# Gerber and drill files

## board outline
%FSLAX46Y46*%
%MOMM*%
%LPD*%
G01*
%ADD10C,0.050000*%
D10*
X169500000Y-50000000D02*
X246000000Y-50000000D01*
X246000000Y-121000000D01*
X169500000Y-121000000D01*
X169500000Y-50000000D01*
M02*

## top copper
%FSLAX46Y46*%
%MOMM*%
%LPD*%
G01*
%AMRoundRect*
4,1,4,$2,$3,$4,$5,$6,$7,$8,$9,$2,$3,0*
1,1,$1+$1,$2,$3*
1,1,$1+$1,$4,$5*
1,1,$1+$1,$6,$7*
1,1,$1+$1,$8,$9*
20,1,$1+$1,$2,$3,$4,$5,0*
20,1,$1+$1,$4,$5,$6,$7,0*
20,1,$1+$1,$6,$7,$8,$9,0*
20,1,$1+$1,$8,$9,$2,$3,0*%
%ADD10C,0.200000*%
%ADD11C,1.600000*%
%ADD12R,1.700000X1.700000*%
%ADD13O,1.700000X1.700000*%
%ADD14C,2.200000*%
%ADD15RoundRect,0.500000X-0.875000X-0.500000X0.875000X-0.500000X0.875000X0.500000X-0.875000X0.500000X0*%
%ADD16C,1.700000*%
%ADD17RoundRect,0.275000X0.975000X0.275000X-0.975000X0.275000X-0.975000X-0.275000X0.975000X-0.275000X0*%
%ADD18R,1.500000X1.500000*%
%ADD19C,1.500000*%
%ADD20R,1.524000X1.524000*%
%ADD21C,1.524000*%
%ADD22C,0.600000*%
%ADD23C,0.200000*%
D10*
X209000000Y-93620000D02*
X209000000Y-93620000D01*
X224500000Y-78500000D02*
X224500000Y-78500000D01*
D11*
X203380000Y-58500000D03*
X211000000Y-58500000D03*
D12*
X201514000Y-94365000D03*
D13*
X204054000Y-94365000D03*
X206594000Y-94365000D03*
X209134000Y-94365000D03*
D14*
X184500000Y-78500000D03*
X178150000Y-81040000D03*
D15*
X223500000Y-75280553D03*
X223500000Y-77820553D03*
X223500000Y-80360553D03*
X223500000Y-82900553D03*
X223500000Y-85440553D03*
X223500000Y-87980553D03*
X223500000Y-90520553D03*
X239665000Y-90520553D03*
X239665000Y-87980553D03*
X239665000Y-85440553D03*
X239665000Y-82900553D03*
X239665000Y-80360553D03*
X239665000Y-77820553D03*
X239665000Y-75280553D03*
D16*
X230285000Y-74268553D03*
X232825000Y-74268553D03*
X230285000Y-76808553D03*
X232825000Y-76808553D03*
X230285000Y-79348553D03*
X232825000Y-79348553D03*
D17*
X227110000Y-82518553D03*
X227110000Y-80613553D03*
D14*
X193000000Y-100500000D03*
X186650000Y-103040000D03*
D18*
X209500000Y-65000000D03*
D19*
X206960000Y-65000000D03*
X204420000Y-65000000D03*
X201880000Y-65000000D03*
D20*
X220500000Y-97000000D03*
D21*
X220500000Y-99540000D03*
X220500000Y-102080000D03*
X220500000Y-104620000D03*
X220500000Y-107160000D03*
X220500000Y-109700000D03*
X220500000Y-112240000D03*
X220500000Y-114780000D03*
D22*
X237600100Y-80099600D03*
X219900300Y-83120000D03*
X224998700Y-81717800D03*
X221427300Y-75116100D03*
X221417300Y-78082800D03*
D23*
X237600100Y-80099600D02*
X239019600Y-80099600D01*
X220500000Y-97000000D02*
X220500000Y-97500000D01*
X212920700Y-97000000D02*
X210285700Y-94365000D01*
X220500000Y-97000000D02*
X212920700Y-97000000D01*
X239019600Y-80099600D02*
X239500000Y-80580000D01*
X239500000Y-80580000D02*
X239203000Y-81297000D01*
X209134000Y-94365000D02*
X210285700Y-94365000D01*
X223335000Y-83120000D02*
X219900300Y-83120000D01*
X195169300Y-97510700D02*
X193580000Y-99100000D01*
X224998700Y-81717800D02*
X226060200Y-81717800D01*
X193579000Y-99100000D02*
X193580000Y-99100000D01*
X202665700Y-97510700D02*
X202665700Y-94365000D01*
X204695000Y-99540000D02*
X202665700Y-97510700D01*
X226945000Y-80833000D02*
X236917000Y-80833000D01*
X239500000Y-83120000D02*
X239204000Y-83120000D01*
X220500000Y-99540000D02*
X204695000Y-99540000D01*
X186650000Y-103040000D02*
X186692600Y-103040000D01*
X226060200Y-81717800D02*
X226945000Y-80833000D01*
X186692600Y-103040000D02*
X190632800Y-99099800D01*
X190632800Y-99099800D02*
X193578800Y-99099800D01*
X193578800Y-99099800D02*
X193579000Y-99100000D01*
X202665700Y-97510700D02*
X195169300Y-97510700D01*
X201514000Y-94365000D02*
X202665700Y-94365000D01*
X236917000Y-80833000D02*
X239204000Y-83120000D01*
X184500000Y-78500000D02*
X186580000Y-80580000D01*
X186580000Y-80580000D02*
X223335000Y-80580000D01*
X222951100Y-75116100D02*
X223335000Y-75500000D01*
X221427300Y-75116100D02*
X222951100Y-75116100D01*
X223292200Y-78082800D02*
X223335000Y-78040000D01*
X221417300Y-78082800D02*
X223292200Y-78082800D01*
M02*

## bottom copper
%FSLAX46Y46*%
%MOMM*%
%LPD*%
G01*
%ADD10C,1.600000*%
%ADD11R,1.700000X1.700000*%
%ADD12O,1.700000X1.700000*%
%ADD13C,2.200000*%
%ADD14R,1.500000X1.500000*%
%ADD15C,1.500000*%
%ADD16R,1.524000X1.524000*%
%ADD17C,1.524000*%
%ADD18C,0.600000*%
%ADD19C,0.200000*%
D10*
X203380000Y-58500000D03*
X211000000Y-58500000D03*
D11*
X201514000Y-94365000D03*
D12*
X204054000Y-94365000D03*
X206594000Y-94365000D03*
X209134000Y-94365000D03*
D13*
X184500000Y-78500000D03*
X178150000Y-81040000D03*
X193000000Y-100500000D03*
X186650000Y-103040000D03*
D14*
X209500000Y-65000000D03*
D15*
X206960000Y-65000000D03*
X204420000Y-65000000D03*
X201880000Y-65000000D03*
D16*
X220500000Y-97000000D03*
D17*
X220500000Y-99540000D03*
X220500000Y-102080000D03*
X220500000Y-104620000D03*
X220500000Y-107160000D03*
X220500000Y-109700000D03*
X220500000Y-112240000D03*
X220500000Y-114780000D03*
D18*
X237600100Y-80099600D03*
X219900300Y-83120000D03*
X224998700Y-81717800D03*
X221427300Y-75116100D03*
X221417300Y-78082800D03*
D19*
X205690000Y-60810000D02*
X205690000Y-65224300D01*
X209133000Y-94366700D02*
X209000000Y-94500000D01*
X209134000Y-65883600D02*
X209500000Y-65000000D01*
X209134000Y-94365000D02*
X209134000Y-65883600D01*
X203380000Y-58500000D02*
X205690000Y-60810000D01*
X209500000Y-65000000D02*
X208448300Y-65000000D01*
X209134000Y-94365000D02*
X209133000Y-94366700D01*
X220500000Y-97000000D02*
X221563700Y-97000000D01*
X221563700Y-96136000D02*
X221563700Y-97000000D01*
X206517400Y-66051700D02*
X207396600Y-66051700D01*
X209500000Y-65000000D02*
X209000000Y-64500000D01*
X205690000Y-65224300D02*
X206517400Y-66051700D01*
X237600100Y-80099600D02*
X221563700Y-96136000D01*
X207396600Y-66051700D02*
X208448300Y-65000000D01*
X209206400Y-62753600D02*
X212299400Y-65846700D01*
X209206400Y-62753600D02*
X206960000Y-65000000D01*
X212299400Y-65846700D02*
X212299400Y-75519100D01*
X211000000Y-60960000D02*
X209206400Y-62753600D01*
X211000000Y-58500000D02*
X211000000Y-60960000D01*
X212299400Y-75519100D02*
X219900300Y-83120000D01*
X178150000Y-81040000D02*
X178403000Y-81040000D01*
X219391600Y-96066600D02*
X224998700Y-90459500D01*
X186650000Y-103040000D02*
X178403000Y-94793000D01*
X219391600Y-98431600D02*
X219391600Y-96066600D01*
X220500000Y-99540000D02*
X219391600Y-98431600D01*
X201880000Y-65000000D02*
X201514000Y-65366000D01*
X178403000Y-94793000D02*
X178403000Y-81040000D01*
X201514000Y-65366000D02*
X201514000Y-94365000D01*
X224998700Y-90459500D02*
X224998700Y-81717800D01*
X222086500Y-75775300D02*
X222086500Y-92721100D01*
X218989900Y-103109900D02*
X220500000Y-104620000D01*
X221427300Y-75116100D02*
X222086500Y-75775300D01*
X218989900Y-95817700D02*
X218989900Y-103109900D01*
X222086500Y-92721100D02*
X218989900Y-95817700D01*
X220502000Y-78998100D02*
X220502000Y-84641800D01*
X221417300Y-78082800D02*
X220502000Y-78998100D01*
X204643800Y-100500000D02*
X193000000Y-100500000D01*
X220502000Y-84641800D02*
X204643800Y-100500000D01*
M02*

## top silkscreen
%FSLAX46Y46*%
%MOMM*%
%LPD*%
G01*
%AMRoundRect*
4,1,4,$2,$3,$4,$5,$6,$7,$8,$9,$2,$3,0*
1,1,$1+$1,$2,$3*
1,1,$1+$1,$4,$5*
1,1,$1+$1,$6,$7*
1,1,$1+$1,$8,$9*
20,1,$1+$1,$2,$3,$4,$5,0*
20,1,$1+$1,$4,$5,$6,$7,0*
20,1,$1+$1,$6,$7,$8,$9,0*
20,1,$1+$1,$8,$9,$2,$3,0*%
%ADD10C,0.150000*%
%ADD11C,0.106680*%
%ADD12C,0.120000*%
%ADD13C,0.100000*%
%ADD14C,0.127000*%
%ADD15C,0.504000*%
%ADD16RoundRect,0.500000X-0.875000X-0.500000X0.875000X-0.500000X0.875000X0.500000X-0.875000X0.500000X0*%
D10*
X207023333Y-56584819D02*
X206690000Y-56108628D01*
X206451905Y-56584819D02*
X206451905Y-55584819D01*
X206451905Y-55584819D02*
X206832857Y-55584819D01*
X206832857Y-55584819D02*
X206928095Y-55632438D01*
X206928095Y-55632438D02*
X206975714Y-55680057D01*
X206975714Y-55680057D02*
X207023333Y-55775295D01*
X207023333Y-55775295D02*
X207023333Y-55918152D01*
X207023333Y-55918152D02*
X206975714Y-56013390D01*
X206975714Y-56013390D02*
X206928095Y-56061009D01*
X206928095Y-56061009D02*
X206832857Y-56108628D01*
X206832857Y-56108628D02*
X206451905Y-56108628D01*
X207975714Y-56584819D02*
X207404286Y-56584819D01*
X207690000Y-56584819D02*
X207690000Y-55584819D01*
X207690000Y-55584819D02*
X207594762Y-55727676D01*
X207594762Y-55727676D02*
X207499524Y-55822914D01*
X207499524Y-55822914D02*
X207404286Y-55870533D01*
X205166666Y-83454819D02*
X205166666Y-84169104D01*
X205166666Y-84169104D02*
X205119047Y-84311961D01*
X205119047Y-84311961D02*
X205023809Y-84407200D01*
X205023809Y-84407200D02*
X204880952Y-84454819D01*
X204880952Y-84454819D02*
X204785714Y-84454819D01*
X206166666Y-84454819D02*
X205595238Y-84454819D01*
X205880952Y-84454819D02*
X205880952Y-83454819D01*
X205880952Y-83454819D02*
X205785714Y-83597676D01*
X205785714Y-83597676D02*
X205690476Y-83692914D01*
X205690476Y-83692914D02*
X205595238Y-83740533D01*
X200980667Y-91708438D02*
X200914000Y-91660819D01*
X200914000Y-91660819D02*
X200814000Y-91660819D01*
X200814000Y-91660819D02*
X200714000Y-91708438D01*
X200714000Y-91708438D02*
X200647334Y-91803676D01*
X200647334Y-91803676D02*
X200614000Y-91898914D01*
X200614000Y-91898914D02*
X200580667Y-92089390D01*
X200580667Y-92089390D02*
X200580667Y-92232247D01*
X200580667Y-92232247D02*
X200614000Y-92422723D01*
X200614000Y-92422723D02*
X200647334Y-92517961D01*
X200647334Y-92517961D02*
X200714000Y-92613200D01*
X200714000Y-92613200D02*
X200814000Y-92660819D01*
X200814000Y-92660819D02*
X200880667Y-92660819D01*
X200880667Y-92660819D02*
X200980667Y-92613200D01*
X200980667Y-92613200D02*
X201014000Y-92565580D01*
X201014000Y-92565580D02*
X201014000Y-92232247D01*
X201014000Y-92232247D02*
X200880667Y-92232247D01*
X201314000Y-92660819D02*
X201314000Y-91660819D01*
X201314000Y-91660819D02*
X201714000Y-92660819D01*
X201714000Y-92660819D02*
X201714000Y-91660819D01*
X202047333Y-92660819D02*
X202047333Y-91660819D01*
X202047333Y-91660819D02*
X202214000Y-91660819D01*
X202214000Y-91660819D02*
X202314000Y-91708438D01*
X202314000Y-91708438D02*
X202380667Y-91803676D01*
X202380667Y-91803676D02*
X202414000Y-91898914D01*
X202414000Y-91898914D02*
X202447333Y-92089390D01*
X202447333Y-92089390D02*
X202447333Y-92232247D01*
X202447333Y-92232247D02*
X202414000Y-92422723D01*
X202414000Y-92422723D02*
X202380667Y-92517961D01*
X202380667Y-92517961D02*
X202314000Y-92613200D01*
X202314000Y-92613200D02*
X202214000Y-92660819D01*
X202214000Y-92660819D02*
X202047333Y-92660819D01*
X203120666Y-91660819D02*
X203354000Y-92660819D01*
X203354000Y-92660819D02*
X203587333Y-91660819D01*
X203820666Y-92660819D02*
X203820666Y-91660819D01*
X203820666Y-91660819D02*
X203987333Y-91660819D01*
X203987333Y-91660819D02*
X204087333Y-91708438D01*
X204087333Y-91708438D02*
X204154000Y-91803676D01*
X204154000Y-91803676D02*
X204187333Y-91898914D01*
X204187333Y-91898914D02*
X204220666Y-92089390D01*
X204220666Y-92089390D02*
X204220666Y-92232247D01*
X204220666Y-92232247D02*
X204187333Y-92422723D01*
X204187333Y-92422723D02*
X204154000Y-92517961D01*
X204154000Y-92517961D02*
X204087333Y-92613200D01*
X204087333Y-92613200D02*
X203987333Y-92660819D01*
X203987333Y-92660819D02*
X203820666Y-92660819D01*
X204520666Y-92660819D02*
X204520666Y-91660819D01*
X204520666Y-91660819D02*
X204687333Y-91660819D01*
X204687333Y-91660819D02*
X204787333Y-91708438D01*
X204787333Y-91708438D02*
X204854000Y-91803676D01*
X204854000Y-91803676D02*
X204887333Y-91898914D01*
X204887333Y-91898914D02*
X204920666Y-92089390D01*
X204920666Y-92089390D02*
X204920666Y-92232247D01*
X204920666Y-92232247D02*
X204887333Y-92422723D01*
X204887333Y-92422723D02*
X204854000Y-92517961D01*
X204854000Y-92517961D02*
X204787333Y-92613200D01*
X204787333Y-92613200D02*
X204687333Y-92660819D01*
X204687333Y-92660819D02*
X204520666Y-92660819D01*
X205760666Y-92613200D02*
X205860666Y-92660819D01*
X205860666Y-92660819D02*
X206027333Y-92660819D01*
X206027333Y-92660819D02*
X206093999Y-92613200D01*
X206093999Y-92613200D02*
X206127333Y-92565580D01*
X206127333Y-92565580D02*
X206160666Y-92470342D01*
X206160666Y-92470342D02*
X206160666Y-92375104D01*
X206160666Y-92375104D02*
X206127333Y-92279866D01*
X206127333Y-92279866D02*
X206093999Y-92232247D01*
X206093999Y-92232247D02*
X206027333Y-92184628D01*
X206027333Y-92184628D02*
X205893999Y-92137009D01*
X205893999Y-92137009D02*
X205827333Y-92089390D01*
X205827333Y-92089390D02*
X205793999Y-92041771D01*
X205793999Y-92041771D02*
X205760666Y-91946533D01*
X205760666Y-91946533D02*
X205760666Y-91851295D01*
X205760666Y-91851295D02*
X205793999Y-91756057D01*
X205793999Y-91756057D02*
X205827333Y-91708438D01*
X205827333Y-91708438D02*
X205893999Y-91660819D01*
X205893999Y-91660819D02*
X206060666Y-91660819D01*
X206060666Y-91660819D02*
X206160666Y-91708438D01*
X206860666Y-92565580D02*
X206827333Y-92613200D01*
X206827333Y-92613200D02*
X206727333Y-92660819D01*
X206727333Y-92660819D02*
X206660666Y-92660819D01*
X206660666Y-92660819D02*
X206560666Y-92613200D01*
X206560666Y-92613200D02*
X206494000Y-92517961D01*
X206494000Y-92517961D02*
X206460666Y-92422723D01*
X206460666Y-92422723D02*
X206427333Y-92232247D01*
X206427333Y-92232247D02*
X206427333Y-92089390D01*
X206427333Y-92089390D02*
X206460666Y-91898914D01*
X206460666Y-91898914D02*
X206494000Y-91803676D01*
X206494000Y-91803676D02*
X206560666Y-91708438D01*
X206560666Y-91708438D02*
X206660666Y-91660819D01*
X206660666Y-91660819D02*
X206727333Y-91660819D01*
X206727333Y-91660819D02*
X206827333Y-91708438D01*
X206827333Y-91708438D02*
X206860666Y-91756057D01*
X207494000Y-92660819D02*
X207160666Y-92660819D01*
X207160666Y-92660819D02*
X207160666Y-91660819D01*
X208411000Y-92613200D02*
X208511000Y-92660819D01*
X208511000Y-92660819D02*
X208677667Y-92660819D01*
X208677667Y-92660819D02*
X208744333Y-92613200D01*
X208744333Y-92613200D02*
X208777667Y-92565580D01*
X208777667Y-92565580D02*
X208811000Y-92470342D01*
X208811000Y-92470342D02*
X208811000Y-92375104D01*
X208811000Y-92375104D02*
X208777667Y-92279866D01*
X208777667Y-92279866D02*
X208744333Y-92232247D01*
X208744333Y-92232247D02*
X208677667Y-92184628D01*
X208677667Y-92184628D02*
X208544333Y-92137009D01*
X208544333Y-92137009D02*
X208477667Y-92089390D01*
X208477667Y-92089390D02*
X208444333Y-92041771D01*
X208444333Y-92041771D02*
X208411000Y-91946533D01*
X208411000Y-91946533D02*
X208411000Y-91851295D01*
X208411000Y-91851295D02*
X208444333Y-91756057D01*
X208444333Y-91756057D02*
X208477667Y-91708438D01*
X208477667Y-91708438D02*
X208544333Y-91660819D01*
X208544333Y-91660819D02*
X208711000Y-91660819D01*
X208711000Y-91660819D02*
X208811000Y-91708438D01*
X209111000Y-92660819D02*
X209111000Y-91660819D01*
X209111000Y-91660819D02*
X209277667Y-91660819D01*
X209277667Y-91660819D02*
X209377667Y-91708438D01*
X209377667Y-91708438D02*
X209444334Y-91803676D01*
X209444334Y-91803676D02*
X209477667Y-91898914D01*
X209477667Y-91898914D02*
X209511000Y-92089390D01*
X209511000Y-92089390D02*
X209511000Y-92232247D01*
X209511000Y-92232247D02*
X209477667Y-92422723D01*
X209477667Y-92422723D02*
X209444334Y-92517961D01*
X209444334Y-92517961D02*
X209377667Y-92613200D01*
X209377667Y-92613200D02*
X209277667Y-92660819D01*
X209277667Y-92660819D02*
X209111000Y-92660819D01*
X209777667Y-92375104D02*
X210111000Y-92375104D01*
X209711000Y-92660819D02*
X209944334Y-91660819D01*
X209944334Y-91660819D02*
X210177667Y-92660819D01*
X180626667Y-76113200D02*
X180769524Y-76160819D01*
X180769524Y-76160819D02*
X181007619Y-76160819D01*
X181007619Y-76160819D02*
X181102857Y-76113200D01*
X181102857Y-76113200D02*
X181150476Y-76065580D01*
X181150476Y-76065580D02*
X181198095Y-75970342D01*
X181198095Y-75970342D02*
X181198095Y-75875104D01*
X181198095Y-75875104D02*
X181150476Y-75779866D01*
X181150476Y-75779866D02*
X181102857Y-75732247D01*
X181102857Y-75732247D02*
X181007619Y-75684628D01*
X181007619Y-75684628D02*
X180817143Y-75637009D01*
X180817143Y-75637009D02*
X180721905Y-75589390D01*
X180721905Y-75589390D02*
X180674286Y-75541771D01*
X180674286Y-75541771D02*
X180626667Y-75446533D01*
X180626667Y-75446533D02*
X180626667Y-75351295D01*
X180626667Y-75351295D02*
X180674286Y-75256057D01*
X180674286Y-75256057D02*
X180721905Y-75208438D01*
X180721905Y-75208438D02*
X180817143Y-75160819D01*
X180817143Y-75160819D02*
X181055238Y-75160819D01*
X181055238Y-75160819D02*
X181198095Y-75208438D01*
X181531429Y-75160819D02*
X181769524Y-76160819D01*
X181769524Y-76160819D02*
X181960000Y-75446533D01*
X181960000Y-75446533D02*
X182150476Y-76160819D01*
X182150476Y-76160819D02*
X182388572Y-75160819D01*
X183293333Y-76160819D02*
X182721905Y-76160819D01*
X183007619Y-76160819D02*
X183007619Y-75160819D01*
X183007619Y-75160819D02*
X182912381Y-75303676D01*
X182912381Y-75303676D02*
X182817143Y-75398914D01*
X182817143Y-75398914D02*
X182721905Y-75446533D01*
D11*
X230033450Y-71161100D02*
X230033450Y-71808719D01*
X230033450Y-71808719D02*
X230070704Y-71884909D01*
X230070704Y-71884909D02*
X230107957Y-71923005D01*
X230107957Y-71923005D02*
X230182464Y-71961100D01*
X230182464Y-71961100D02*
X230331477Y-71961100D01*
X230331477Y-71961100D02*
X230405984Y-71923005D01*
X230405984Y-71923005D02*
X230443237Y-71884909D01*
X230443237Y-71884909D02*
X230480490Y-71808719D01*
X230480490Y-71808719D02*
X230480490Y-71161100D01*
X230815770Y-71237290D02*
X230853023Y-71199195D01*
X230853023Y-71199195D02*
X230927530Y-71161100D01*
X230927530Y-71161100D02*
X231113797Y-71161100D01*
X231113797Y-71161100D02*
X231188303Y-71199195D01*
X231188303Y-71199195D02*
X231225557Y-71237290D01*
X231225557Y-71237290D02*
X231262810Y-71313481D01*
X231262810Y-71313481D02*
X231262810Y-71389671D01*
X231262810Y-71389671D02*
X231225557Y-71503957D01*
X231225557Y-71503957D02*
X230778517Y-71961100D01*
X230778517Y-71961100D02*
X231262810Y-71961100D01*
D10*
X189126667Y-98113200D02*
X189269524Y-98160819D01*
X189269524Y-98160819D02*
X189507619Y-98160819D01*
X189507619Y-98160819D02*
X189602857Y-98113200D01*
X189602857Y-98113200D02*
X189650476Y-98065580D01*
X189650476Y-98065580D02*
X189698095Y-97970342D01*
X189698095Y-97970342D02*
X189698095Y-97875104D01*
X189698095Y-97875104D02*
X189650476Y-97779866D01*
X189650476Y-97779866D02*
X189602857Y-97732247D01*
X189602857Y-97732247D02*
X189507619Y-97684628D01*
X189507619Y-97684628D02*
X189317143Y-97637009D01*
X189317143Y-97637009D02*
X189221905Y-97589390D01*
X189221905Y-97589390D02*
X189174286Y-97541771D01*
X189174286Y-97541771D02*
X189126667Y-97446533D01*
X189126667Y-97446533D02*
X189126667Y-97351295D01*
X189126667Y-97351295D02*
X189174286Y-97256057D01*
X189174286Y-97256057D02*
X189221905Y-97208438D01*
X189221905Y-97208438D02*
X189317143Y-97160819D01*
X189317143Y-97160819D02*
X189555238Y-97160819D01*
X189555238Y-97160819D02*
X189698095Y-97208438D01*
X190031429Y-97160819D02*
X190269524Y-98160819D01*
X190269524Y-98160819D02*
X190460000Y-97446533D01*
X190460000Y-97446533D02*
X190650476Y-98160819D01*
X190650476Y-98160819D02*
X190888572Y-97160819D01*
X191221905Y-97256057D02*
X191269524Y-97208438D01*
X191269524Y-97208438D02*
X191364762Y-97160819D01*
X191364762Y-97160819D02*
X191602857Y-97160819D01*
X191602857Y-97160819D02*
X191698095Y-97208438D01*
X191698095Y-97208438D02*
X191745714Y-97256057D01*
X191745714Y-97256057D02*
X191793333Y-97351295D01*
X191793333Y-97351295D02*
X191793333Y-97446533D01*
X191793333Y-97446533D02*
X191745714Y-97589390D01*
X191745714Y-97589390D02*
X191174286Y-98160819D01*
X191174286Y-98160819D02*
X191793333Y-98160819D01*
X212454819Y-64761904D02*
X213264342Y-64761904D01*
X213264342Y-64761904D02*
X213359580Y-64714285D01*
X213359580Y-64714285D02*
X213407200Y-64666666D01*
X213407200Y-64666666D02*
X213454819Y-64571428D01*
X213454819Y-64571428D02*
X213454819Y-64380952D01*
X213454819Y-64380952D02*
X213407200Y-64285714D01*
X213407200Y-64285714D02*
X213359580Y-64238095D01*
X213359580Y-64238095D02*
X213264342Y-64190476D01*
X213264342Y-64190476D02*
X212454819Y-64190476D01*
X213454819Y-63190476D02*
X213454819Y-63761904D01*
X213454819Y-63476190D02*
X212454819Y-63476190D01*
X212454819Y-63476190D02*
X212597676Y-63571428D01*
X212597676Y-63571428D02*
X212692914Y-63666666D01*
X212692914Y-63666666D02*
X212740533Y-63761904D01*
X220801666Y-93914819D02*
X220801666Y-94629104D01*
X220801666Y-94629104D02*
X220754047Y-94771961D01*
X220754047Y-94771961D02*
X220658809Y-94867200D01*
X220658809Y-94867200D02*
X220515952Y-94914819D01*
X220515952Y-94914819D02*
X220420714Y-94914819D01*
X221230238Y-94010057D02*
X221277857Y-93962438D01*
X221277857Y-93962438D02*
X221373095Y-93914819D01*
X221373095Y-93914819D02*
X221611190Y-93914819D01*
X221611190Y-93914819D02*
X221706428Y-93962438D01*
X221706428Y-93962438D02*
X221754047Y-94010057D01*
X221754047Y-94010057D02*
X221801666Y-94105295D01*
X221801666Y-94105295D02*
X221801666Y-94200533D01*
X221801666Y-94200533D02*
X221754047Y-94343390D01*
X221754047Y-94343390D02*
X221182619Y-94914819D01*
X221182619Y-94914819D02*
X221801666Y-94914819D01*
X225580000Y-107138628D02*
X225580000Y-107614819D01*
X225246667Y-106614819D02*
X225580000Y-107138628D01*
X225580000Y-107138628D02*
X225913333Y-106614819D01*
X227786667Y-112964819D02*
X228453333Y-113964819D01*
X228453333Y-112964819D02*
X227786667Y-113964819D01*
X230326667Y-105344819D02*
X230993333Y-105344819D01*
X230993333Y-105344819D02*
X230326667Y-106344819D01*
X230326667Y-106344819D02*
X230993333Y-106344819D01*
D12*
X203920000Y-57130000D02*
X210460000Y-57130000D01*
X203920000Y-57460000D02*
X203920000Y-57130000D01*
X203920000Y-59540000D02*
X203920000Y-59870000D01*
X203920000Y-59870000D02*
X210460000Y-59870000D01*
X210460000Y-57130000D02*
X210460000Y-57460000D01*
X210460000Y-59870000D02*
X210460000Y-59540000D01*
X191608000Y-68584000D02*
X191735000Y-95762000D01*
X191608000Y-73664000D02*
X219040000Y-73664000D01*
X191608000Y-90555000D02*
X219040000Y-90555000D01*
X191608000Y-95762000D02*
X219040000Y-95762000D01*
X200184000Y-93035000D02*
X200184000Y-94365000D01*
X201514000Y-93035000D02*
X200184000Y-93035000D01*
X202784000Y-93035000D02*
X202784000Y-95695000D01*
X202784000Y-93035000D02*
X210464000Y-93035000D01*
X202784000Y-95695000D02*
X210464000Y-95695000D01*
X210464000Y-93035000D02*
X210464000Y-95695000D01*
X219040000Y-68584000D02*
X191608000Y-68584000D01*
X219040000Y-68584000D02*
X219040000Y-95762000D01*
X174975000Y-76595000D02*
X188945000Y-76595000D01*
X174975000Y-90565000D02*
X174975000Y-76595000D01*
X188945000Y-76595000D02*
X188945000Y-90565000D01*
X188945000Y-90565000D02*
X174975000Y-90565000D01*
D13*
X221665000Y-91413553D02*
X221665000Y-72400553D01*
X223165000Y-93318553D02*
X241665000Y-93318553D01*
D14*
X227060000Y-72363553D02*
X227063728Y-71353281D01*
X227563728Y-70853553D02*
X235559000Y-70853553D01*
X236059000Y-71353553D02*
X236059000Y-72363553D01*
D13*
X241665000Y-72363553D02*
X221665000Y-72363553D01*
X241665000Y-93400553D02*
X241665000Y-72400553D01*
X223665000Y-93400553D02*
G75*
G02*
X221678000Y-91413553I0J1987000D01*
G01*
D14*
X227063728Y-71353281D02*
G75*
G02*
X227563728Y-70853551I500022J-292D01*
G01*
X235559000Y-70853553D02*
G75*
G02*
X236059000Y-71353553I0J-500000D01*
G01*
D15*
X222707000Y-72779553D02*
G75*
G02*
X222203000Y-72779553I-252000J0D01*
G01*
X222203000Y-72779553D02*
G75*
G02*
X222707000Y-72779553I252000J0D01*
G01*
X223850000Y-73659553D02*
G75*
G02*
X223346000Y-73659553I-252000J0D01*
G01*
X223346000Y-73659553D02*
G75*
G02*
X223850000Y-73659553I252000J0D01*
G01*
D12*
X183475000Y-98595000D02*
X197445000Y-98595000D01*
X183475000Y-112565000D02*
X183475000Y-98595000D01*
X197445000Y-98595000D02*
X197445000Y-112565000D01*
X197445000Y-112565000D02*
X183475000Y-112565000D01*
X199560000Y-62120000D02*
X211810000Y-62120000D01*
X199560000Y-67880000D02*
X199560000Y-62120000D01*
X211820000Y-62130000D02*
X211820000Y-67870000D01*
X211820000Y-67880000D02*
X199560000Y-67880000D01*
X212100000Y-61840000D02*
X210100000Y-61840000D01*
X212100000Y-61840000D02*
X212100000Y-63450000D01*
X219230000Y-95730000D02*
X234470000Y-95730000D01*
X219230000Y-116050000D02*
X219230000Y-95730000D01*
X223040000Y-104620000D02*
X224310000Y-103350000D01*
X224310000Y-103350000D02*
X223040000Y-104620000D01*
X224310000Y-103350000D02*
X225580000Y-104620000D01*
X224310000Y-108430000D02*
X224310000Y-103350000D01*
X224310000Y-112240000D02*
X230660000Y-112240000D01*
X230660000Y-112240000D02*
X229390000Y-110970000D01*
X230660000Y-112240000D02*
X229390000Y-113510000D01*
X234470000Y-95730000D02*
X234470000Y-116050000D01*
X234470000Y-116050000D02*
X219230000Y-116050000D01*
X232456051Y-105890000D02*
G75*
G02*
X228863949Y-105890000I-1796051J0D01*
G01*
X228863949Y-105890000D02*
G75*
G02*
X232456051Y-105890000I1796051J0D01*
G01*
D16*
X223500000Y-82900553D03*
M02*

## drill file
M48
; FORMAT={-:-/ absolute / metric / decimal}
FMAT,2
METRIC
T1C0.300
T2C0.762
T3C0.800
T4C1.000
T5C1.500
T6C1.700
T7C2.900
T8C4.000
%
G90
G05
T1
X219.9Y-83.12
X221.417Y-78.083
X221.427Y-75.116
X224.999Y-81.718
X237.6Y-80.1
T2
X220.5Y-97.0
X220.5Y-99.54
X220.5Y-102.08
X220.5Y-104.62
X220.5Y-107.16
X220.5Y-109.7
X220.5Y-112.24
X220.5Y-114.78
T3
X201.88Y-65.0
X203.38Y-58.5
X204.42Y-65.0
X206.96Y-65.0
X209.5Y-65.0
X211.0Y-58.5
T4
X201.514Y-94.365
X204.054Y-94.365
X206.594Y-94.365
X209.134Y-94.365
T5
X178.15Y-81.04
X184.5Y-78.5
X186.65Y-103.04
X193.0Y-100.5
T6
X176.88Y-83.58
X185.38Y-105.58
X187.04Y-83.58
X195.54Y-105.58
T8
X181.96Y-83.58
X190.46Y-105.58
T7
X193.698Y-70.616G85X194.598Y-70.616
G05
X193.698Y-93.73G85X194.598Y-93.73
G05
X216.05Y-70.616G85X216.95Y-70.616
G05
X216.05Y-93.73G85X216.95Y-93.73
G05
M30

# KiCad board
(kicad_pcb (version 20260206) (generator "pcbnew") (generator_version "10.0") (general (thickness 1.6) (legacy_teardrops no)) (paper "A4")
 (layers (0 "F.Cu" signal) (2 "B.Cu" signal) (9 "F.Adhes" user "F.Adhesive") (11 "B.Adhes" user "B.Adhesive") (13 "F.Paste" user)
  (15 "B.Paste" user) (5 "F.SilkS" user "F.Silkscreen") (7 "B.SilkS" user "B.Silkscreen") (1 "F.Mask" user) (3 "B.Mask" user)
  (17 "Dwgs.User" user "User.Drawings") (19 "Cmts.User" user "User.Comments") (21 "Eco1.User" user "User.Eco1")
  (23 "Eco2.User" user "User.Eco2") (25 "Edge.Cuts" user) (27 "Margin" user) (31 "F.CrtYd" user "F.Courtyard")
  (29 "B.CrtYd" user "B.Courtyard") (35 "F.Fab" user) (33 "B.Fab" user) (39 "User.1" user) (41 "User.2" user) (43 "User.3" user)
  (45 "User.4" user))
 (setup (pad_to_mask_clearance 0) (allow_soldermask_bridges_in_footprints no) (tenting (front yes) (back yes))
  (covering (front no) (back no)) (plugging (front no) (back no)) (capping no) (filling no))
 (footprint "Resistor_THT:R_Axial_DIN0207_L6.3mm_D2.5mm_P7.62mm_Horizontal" (layer "F.Cu") (at 203.38 58.5)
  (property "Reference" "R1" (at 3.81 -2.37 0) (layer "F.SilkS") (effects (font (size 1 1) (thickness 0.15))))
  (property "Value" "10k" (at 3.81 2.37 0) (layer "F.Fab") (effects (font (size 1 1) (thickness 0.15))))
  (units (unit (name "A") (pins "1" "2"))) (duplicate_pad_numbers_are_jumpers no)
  (fp_line (start 0.54 -1.37) (end 7.08 -1.37) (stroke (width 0.12) (type solid)) (layer "F.SilkS"))
  (fp_line (start 0.54 -1.04) (end 0.54 -1.37) (stroke (width 0.12) (type solid)) (layer "F.SilkS"))
  (fp_line (start 0.54 1.04) (end 0.54 1.37) (stroke (width 0.12) (type solid)) (layer "F.SilkS"))
  (fp_line (start 0.54 1.37) (end 7.08 1.37) (stroke (width 0.12) (type solid)) (layer "F.SilkS"))
  (fp_line (start 7.08 -1.37) (end 7.08 -1.04) (stroke (width 0.12) (type solid)) (layer "F.SilkS"))
  (fp_line (start 7.08 1.37) (end 7.08 1.04) (stroke (width 0.12) (type solid)) (layer "F.SilkS"))
  (pad "1" thru_hole circle (at 0 0) (size 1.6 1.6) (drill 0.8) (layers "*.Cu" "*.Mask") (remove_unused_layers no) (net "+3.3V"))
  (pad "2" thru_hole circle (at 7.62 0) (size 1.6 1.6) (drill 0.8) (layers "*.Cu" "*.Mask") (remove_unused_layers no) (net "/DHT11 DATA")))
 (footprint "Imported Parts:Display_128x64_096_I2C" (layer "F.Cu") (at 205.324 70.365)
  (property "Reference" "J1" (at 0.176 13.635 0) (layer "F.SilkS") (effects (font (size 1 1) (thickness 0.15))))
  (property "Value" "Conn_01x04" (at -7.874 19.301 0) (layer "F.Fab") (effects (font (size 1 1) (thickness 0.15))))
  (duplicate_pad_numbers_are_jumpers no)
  (fp_line (start -13.716 -1.781) (end -13.589 25.397) (stroke (width 0.12) (type solid)) (layer "F.SilkS"))
  (fp_line (start -13.716 3.299) (end 13.716 3.299) (stroke (width 0.12) (type solid)) (layer "F.SilkS"))
  (fp_line (start -13.716 20.19) (end 13.716 20.19) (stroke (width 0.12) (type solid)) (layer "F.SilkS"))
  (fp_line (start -13.716 25.397) (end 13.716 25.397) (stroke (width 0.12) (type solid)) (layer "F.SilkS"))
  (fp_line (start -5.14 22.67) (end -5.14 24) (stroke (width 0.12) (type solid)) (layer "F.SilkS"))
  (fp_line (start -3.81 22.67) (end -5.14 22.67) (stroke (width 0.12) (type solid)) (layer "F.SilkS"))
  (fp_line (start -2.54 22.67) (end -2.54 25.33) (stroke (width 0.12) (type solid)) (layer "F.SilkS"))
  (fp_line (start -2.54 22.67) (end 5.14 22.67) (stroke (width 0.12) (type solid)) (layer "F.SilkS"))
  (fp_line (start -2.54 25.33) (end 5.14 25.33) (stroke (width 0.12) (type solid)) (layer "F.SilkS"))
  (fp_line (start 5.14 22.67) (end 5.14 25.33) (stroke (width 0.12) (type solid)) (layer "F.SilkS"))
  (fp_line (start 13.716 -1.781) (end -13.716 -1.781) (stroke (width 0.12) (type solid)) (layer "F.SilkS"))
  (fp_line (start 13.716 -1.781) (end 13.716 25.397) (stroke (width 0.12) (type solid)) (layer "F.SilkS"))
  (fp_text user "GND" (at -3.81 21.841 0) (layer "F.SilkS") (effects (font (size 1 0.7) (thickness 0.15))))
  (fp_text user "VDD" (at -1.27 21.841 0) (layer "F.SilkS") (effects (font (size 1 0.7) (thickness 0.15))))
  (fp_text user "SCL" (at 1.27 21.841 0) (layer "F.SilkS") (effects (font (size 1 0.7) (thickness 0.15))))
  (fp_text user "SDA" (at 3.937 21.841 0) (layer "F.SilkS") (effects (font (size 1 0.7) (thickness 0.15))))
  (pad "" np_thru_hole oval (at -11.176 0.251) (size 3.8 2.9) (drill oval 3.8 2.9) (layers "*.Cu" "*.Mask"))
  (pad "" np_thru_hole oval (at -11.176 23.365) (size 3.8 2.9) (drill oval 3.8 2.9) (layers "*.Cu" "*.Mask"))
  (pad "" np_thru_hole oval (at 11.176 0.251) (size 3.8 2.9) (drill oval 3.8 2.9) (layers "*.Cu" "*.Mask"))
  (pad "" np_thru_hole oval (at 11.176 23.365) (size 3.8 2.9) (drill oval 3.8 2.9) (layers "*.Cu" "*.Mask"))
  (pad "1" thru_hole rect (at -3.81 24 270) (size 1.7 1.7) (drill 1) (layers "*.Cu" "*.Mask") (remove_unused_layers no) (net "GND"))
  (pad "2" thru_hole oval (at -1.27 24 270) (size 1.7 1.7) (drill 1) (layers "*.Cu" "*.Mask") (remove_unused_layers no)
   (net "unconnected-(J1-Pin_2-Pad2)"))
  (pad "3" thru_hole oval (at 1.27 24 270) (size 1.7 1.7) (drill 1) (layers "*.Cu" "*.Mask") (remove_unused_layers no)
   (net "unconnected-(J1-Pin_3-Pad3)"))
  (pad "4" thru_hole oval (at 3.81 24 270) (size 1.7 1.7) (drill 1) (layers "*.Cu" "*.Mask") (remove_unused_layers no) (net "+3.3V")))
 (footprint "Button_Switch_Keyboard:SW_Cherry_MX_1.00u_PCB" (layer "F.Cu") (at 184.5 78.5)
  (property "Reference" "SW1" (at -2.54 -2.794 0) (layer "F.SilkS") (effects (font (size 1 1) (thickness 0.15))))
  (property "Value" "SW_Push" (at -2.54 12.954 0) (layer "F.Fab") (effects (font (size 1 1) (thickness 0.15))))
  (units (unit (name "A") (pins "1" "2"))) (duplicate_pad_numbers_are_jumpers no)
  (fp_line (start -9.525 -1.905) (end 4.445 -1.905) (stroke (width 0.12) (type solid)) (layer "F.SilkS"))
  (fp_line (start -9.525 12.065) (end -9.525 -1.905) (stroke (width 0.12) (type solid)) (layer "F.SilkS"))
  (fp_line (start 4.445 -1.905) (end 4.445 12.065) (stroke (width 0.12) (type solid)) (layer "F.SilkS"))
  (fp_line (start 4.445 12.065) (end -9.525 12.065) (stroke (width 0.12) (type solid)) (layer "F.SilkS"))
  (pad "" np_thru_hole circle (at -7.62 5.08) (size 1.7 1.7) (drill 1.7) (layers "*.Cu" "*.Mask"))
  (pad "" np_thru_hole circle (at -2.54 5.08) (size 4 4) (drill 4) (layers "*.Cu" "*.Mask"))
  (pad "" np_thru_hole circle (at 2.54 5.08) (size 1.7 1.7) (drill 1.7) (layers "*.Cu" "*.Mask"))
  (pad "1" thru_hole circle (at 0 0) (size 2.2 2.2) (drill 1.5) (layers "*.Cu" "*.Mask") (remove_unused_layers no) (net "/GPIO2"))
  (pad "2" thru_hole circle (at -6.35 2.54) (size 2.2 2.2) (drill 1.5) (layers "*.Cu" "*.Mask") (remove_unused_layers no) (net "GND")))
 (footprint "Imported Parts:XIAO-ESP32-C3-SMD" (layer "F.Cu") (at 222.665 93.400553)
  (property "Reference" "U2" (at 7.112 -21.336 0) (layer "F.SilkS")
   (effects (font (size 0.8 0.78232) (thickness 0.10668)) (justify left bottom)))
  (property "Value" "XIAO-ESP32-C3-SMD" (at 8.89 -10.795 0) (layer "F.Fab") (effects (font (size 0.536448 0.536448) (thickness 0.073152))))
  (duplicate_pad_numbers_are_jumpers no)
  (fp_line (start -1 -1.987) (end -1 -21) (stroke (width 0.1) (type solid)) (layer "F.SilkS"))
  (fp_line (start 0.5 -0.082) (end 19 -0.082) (stroke (width 0.1) (type solid)) (layer "F.SilkS"))
  (fp_line (start 4.395 -21.037) (end 4.398728 -22.047272) (stroke (width 0.127) (type solid)) (layer "F.SilkS"))
  (fp_line (start 4.898728 -22.547) (end 12.894 -22.547) (stroke (width 0.127) (type solid)) (layer "F.SilkS"))
  (fp_line (start 13.394 -22.047) (end 13.394 -21.037) (stroke (width 0.127) (type solid)) (layer "F.SilkS"))
  (fp_line (start 19 -21.037) (end -1 -21.037) (stroke (width 0.1) (type solid)) (layer "F.SilkS"))
  (fp_line (start 19 0) (end 19 -21) (stroke (width 0.1) (type solid)) (layer "F.SilkS"))
  (fp_arc (start 1 0) (mid -0.405021 -0.581979) (end -0.987 -1.987) (stroke (width 0.1) (type solid)) (layer "F.SilkS"))
  (fp_arc (start 4.398728 -22.047272) (mid 4.545272 -22.40064) (end 4.898728 -22.547) (stroke (width 0.127) (type default))
   (layer "F.SilkS"))
  (fp_arc (start 12.894 -22.547) (mid 13.247553 -22.400553) (end 13.394 -22.047) (stroke (width 0.127) (type default)) (layer "F.SilkS"))
  (fp_circle (center -0.21 -20.621) (end -0.21 -20.875) (stroke (width 0.5) (type solid)) (fill yes) (layer "F.SilkS"))
  (fp_circle (center 0.933 -19.741) (end 0.933 -19.995) (stroke (width 0.5) (type solid)) (fill yes) (layer "F.SilkS"))
  (pad "1" smd roundrect (at 0.835 -18.12) (size 2.75 2) (layers "F.Cu" "F.Mask" "F.Paste") (roundrect_rratio 0.25) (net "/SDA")
   (solder_mask_margin 0.0508) (thermal_bridge_angle 45))
  (pad "2" smd roundrect (at 0.835 -15.58) (size 2.75 2) (layers "F.Cu" "F.Mask" "F.Paste") (roundrect_rratio 0.25) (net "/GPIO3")
   (solder_mask_margin 0.0508) (thermal_bridge_angle 45))
  (pad "3" smd roundrect (at 0.835 -13.04) (size 2.75 2) (layers "F.Cu" "F.Mask" "F.Paste") (roundrect_rratio 0.25) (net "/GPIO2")
   (solder_mask_margin 0.0508) (thermal_bridge_angle 45))
  (pad "4" smd roundrect (at 0.835 -10.5) (size 2.75 2) (layers "F.Cu" "F.Mask" "F.SilkS" "F.Paste") (roundrect_rratio 0.25)
   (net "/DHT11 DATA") (solder_mask_margin 0.0508) (clearance 0.2) (thermal_bridge_angle 45))
  (pad "5" smd roundrect (at 0.835 -7.96) (size 2.75 2) (layers "F.Cu" "F.Mask" "F.Paste") (roundrect_rratio 0.25)
   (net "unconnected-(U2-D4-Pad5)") (solder_mask_margin 0.0508) (thermal_bridge_angle 45))
  (pad "6" smd roundrect (at 0.835 -5.42) (size 2.75 2) (layers "F.Cu" "F.Mask" "F.Paste") (roundrect_rratio 0.25)
   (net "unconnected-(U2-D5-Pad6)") (solder_mask_margin 0.0508) (thermal_bridge_angle 45))
  (pad "7" smd roundrect (at 0.835 -2.88) (size 2.75 2) (layers "F.Cu" "F.Mask" "F.Paste") (roundrect_rratio 0.25)
   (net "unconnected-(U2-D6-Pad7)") (solder_mask_margin 0.0508) (thermal_bridge_angle 45))
  (pad "8" smd roundrect (at 17 -2.88) (size 2.75 2) (layers "F.Cu" "F.Mask" "F.Paste") (roundrect_rratio 0.25)
   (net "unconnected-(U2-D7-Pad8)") (solder_mask_margin 0.0508) (thermal_bridge_angle 45))
  (pad "9" smd roundrect (at 17 -5.42) (size 2.75 2) (layers "F.Cu" "F.Mask" "F.Paste") (roundrect_rratio 0.25)
   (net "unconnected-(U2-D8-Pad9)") (solder_mask_margin 0.0508) (thermal_bridge_angle 45))
  (pad "10" smd roundrect (at 17 -7.96) (size 2.75 2) (layers "F.Cu" "F.Mask" "F.Paste") (roundrect_rratio 0.25) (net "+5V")
   (solder_mask_margin 0.0508) (thermal_bridge_angle 45))
  (pad "11" smd roundrect (at 17 -10.5) (size 2.75 2) (layers "F.Cu" "F.Mask" "F.Paste") (roundrect_rratio 0.25) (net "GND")
   (solder_mask_margin 0.0508) (thermal_bridge_angle 45))
  (pad "12" smd roundrect (at 17 -13.04) (size 2.75 2) (layers "F.Cu" "F.Mask" "F.Paste") (roundrect_rratio 0.25) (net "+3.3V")
   (solder_mask_margin 0.0508) (thermal_bridge_angle 45))
  (pad "13" smd roundrect (at 17 -15.58) (size 2.75 2) (layers "F.Cu" "F.Mask" "F.Paste") (roundrect_rratio 0.25)
   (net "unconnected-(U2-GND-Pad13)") (solder_mask_margin 0.0508) (thermal_bridge_angle 45))
  (pad "14" smd roundrect (at 17 -18.12) (size 2.75 2) (layers "F.Cu" "F.Mask" "F.Paste") (roundrect_rratio 0.25)
   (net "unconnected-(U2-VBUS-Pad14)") (solder_mask_margin 0.0508) (thermal_bridge_angle 45))
  (pad "15" smd circle (at 7.62 -19.132) (size 1.7 1.7) (layers "F.Cu" "F.Mask" "F.Paste") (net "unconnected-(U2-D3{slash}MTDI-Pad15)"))
  (pad "16" smd circle (at 10.16 -19.132) (size 1.7 1.7) (layers "F.Cu" "F.Mask" "F.Paste") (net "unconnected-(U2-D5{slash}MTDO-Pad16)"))
  (pad "17" smd circle (at 7.62 -16.592) (size 1.7 1.7) (layers "F.Cu" "F.Mask" "F.Paste") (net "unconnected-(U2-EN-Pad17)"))
  (pad "18" smd circle (at 10.16 -16.592) (size 1.7 1.7) (layers "F.Cu" "F.Mask" "F.Paste") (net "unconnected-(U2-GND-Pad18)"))
  (pad "19" smd circle (at 7.62 -14.052) (size 1.7 1.7) (layers "F.Cu" "F.Mask" "F.Paste") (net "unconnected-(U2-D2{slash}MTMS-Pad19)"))
  (pad "20" smd circle (at 10.16 -14.052) (size 1.7 1.7) (layers "F.Cu" "F.Mask" "F.Paste") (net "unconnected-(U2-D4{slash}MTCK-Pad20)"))
  (pad "21" smd roundrect (at 4.445 -10.882 180) (size 2.5 1.1) (layers "F.Cu" "F.Mask" "F.Paste") (roundrect_rratio 0.25)
   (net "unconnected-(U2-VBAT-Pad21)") (thermal_bridge_angle 45))
  (pad "22" smd roundrect (at 4.445 -12.787 180) (size 2.5 1.1) (layers "F.Cu" "F.Mask" "F.Paste") (roundrect_rratio 0.25) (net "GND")
   (thermal_bridge_angle 45)))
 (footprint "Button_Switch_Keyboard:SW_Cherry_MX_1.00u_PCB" (layer "F.Cu") (at 193 100.5)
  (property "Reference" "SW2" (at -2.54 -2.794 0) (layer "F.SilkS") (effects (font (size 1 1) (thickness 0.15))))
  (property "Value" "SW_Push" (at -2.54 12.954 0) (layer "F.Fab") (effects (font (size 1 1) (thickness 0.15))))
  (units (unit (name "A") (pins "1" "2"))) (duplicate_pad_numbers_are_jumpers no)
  (fp_line (start -9.525 -1.905) (end 4.445 -1.905) (stroke (width 0.12) (type solid)) (layer "F.SilkS"))
  (fp_line (start -9.525 12.065) (end -9.525 -1.905) (stroke (width 0.12) (type solid)) (layer "F.SilkS"))
  (fp_line (start 4.445 -1.905) (end 4.445 12.065) (stroke (width 0.12) (type solid)) (layer "F.SilkS"))
  (fp_line (start 4.445 12.065) (end -9.525 12.065) (stroke (width 0.12) (type solid)) (layer "F.SilkS"))
  (pad "" np_thru_hole circle (at -7.62 5.08) (size 1.7 1.7) (drill 1.7) (layers "*.Cu" "*.Mask"))
  (pad "" np_thru_hole circle (at -2.54 5.08) (size 4 4) (drill 4) (layers "*.Cu" "*.Mask"))
  (pad "" np_thru_hole circle (at 2.54 5.08) (size 1.7 1.7) (drill 1.7) (layers "*.Cu" "*.Mask"))
  (pad "1" thru_hole circle (at 0 0) (size 2.2 2.2) (drill 1.5) (layers "*.Cu" "*.Mask") (remove_unused_layers no) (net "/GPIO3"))
  (pad "2" thru_hole circle (at -6.35 2.54) (size 2.2 2.2) (drill 1.5) (layers "*.Cu" "*.Mask") (remove_unused_layers no) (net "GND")))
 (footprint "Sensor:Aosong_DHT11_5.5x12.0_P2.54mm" (layer "F.Cu") (at 209.5 65 -90)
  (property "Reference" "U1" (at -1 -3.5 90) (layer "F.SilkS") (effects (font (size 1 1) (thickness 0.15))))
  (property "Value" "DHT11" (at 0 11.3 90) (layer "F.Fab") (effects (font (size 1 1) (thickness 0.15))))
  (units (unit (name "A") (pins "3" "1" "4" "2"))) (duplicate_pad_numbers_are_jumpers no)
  (fp_line (start -2.88 9.94) (end -2.88 -2.31) (stroke (width 0.12) (type solid)) (layer "F.SilkS"))
  (fp_line (start 2.88 9.94) (end -2.88 9.94) (stroke (width 0.12) (type solid)) (layer "F.SilkS"))
  (fp_line (start -2.87 -2.32) (end 2.87 -2.32) (stroke (width 0.12) (type solid)) (layer "F.SilkS"))
  (fp_line (start 2.88 -2.32) (end 2.88 9.94) (stroke (width 0.12) (type solid)) (layer "F.SilkS"))
  (fp_line (start -3.16 -2.6) (end -3.16 -0.6) (stroke (width 0.12) (type solid)) (layer "F.SilkS"))
  (fp_line (start -3.16 -2.6) (end -1.55 -2.6) (stroke (width 0.12) (type solid)) (layer "F.SilkS"))
  (pad "1" thru_hole rect (at 0 0 270) (size 1.5 1.5) (drill 0.8) (layers "*.Cu" "*.Mask") (remove_unused_layers no) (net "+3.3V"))
  (pad "2" thru_hole circle (at 0 2.54 270) (size 1.5 1.5) (drill 0.8) (layers "*.Cu" "*.Mask") (remove_unused_layers no)
   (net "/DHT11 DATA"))
  (pad "3" thru_hole circle (at 0 5.08 270) (size 1.5 1.5) (drill 0.8) (layers "*.Cu" "*.Mask") (remove_unused_layers no)
   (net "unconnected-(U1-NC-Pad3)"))
  (pad "4" thru_hole circle (at 0 7.62 270) (size 1.5 1.5) (drill 0.8) (layers "*.Cu" "*.Mask") (remove_unused_layers no) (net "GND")))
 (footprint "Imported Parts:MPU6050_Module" (layer "F.Cu") (at 220.5 97)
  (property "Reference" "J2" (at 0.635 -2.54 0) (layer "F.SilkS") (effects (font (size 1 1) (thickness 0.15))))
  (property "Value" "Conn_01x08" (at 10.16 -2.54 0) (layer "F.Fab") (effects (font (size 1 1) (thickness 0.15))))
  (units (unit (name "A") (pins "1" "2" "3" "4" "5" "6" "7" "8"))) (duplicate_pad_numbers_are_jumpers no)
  (fp_line (start -1.27 -1.27) (end 13.97 -1.27) (stroke (width 0.12) (type solid)) (layer "F.SilkS"))
  (fp_line (start -1.27 19.05) (end -1.27 -1.27) (stroke (width 0.12) (type solid)) (layer "F.SilkS"))
  (fp_line (start 2.54 7.62) (end 3.81 6.35) (stroke (width 0.12) (type solid)) (layer "F.SilkS"))
  (fp_line (start 3.81 6.35) (end 2.54 7.62) (stroke (width 0.12) (type solid)) (layer "F.SilkS"))
  (fp_line (start 3.81 6.35) (end 5.08 7.62) (stroke (width 0.12) (type solid)) (layer "F.SilkS"))
  (fp_line (start 3.81 11.43) (end 3.81 6.35) (stroke (width 0.12) (type solid)) (layer "F.SilkS"))
  (fp_line (start 3.81 15.24) (end 10.16 15.24) (stroke (width 0.12) (type solid)) (layer "F.SilkS"))
  (fp_line (start 10.16 15.24) (end 8.89 13.97) (stroke (width 0.12) (type solid)) (layer "F.SilkS"))
  (fp_line (start 10.16 15.24) (end 8.89 16.51) (stroke (width 0.12) (type solid)) (layer "F.SilkS"))
  (fp_line (start 13.97 -1.27) (end 13.97 19.05) (stroke (width 0.12) (type solid)) (layer "F.SilkS"))
  (fp_line (start 13.97 19.05) (end -1.27 19.05) (stroke (width 0.12) (type solid)) (layer "F.SilkS"))
  (fp_circle (center 10.16 8.89) (end 8.89 7.62) (stroke (width 0.12) (type solid)) (fill no) (layer "F.SilkS"))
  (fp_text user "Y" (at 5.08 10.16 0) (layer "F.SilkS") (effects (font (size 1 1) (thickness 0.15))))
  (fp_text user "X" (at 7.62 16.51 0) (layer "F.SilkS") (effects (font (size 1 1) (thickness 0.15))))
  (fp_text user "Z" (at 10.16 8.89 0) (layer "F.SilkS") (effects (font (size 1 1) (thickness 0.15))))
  (pad "1" thru_hole rect (at 0 0) (size 1.524 1.524) (drill 0.762) (layers "*.Cu" "*.Mask") (remove_unused_layers no) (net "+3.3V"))
  (pad "2" thru_hole circle (at 0 2.54) (size 1.524 1.524) (drill 0.762) (layers "*.Cu" "*.Mask") (remove_unused_layers no) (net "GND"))
  (pad "3" thru_hole circle (at 0 5.08) (size 1.524 1.524) (drill 0.762) (layers "*.Cu" "*.Mask") (remove_unused_layers no) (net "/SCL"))
  (pad "4" thru_hole circle (at 0 7.62) (size 1.524 1.524) (drill 0.762) (layers "*.Cu" "*.Mask") (remove_unused_layers no) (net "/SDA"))
  (pad "5" thru_hole circle (at 0 10.16) (size 1.524 1.524) (drill 0.762) (layers "*.Cu" "*.Mask") (remove_unused_layers no)
   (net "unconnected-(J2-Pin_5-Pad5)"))
  (pad "6" thru_hole circle (at 0 12.7) (size 1.524 1.524) (drill 0.762) (layers "*.Cu" "*.Mask") (remove_unused_layers no)
   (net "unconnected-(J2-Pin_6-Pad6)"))
  (pad "7" thru_hole circle (at 0 15.24) (size 1.524 1.524) (drill 0.762) (layers "*.Cu" "*.Mask") (remove_unused_layers no)
   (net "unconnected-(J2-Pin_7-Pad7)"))
  (pad "8" thru_hole circle (at 0 17.78) (size 1.524 1.524) (drill 0.762) (layers "*.Cu" "*.Mask") (remove_unused_layers no)
   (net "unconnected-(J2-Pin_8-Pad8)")))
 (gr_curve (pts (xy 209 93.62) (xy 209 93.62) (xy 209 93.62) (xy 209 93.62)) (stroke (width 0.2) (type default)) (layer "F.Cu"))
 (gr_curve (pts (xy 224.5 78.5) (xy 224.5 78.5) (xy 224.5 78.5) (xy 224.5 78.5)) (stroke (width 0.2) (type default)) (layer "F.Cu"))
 (gr_rect (start 169.5 50) (end 246 121) (stroke (width 0.05) (type default)) (fill no) (layer "Edge.Cuts"))
 (segment (start 237.6001 80.0996) (end 239.0196 80.0996) (width 0.2) (layer "F.Cu") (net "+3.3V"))
 (segment (start 220.5 97) (end 220.5 97.5) (width 0.2) (layer "F.Cu") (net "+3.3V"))
 (segment (start 212.9207 97) (end 210.2857 94.365) (width 0.2) (layer "F.Cu") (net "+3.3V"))
 (segment (start 220.5 97) (end 212.9207 97) (width 0.2) (layer "F.Cu") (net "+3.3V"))
 (segment (start 239.0196 80.0996) (end 239.5 80.58) (width 0.2) (layer "F.Cu") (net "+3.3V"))
 (segment (start 239.5 80.58) (end 239.203 81.297) (width 0.2) (layer "F.Cu") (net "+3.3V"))
 (segment (start 209.134 94.365) (end 210.2857 94.365) (width 0.2) (layer "F.Cu") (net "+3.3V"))
 (via (at 237.6001 80.0996) (size 0.6) (drill 0.3) (layers "F.Cu" "B.Cu") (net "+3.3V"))
 (segment (start 205.69 60.81) (end 205.69 65.2243) (width 0.2) (layer "B.Cu") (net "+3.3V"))
 (segment (start 209.133 94.3667) (end 209 94.5) (width 0.2) (layer "B.Cu") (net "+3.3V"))
 (segment (start 209.134 65.8836) (end 209.5 65) (width 0.2) (layer "B.Cu") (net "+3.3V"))
 (segment (start 209.134 94.365) (end 209.134 65.8836) (width 0.2) (layer "B.Cu") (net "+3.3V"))
 (segment (start 203.38 58.5) (end 205.69 60.81) (width 0.2) (layer "B.Cu") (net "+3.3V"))
 (segment (start 209.5 65) (end 208.4483 65) (width 0.2) (layer "B.Cu") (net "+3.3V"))
 (segment (start 209.134 94.365) (end 209.133 94.3667) (width 0.2) (layer "B.Cu") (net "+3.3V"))
 (segment (start 220.5 97) (end 221.5637 97) (width 0.2) (layer "B.Cu") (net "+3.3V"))
 (segment (start 221.5637 96.136) (end 221.5637 97) (width 0.2) (layer "B.Cu") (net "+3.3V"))
 (segment (start 206.5174 66.0517) (end 207.3966 66.0517) (width 0.2) (layer "B.Cu") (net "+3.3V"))
 (segment (start 209.5 65) (end 209 64.5) (width 0.2) (layer "B.Cu") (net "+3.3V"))
 (segment (start 205.69 65.2243) (end 206.5174 66.0517) (width 0.2) (layer "B.Cu") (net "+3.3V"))
 (segment (start 237.6001 80.0996) (end 221.5637 96.136) (width 0.2) (layer "B.Cu") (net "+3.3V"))
 (segment (start 207.3966 66.0517) (end 208.4483 65) (width 0.2) (layer "B.Cu") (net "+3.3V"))
 (segment (start 223.335 83.12) (end 219.9003 83.12) (width 0.2) (layer "F.Cu") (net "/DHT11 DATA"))
 (via (at 219.9003 83.12) (size 0.6) (drill 0.3) (layers "F.Cu" "B.Cu") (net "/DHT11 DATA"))
 (segment (start 209.2064 62.7536) (end 212.2994 65.8467) (width 0.2) (layer "B.Cu") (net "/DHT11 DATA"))
 (segment (start 209.2064 62.7536) (end 206.96 65) (width 0.2) (layer "B.Cu") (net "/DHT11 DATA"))
 (segment (start 212.2994 65.8467) (end 212.2994 75.5191) (width 0.2) (layer "B.Cu") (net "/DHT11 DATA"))
 (segment (start 211 60.96) (end 209.2064 62.7536) (width 0.2) (layer "B.Cu") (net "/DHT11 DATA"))
 (segment (start 211 58.5) (end 211 60.96) (width 0.2) (layer "B.Cu") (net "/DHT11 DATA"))
 (segment (start 212.2994 75.5191) (end 219.9003 83.12) (width 0.2) (layer "B.Cu") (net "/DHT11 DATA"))
 (segment (start 195.1693 97.5107) (end 193.58 99.1) (width 0.2) (layer "F.Cu") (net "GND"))
 (segment (start 224.9987 81.7178) (end 226.0602 81.7178) (width 0.2) (layer "F.Cu") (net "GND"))
 (segment (start 193.579 99.1) (end 193.58 99.1) (width 0.2) (layer "F.Cu") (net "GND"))
 (segment (start 202.6657 97.5107) (end 202.6657 94.365) (width 0.2) (layer "F.Cu") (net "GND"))
 (segment (start 204.695 99.54) (end 202.6657 97.5107) (width 0.2) (layer "F.Cu") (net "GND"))
 (segment (start 226.945 80.833) (end 236.917 80.833) (width 0.2) (layer "F.Cu") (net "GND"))
 (segment (start 239.5 83.12) (end 239.204 83.12) (width 0.2) (layer "F.Cu") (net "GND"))
 (segment (start 220.5 99.54) (end 204.695 99.54) (width 0.2) (layer "F.Cu") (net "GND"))
 (segment (start 186.65 103.04) (end 186.6926 103.04) (width 0.2) (layer "F.Cu") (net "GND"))
 (segment (start 226.0602 81.7178) (end 226.945 80.833) (width 0.2) (layer "F.Cu") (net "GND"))
 (segment (start 186.6926 103.04) (end 190.6328 99.0998) (width 0.2) (layer "F.Cu") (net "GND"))
 (segment (start 190.6328 99.0998) (end 193.5788 99.0998) (width 0.2) (layer "F.Cu") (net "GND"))
 (segment (start 193.5788 99.0998) (end 193.579 99.1) (width 0.2) (layer "F.Cu") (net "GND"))
 (segment (start 202.6657 97.5107) (end 195.1693 97.5107) (width 0.2) (layer "F.Cu") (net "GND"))
 (segment (start 201.514 94.365) (end 202.6657 94.365) (width 0.2) (layer "F.Cu") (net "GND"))
 (segment (start 236.917 80.833) (end 239.204 83.12) (width 0.2) (layer "F.Cu") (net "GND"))
 (via (at 224.9987 81.7178) (size 0.6) (drill 0.3) (layers "F.Cu" "B.Cu") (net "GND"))
 (segment (start 178.15 81.04) (end 178.403 81.04) (width 0.2) (layer "B.Cu") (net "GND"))
 (segment (start 219.3916 96.0666) (end 224.9987 90.4595) (width 0.2) (layer "B.Cu") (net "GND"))
 (segment (start 186.65 103.04) (end 178.403 94.793) (width 0.2) (layer "B.Cu") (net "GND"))
 (segment (start 219.3916 98.4316) (end 219.3916 96.0666) (width 0.2) (layer "B.Cu") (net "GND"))
 (segment (start 220.5 99.54) (end 219.3916 98.4316) (width 0.2) (layer "B.Cu") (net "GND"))
 (segment (start 201.88 65) (end 201.514 65.366) (width 0.2) (layer "B.Cu") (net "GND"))
 (segment (start 178.403 94.793) (end 178.403 81.04) (width 0.2) (layer "B.Cu") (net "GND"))
 (segment (start 201.514 65.366) (end 201.514 94.365) (width 0.2) (layer "B.Cu") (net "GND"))
 (segment (start 224.9987 90.4595) (end 224.9987 81.7178) (width 0.2) (layer "B.Cu") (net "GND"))
 (segment (start 184.5 78.5) (end 186.58 80.58) (width 0.2) (layer "F.Cu") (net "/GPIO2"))
 (segment (start 186.58 80.58) (end 223.335 80.58) (width 0.2) (layer "F.Cu") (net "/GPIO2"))
 (segment (start 222.9511 75.1161) (end 223.335 75.5) (width 0.2) (layer "F.Cu") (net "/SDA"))
 (segment (start 221.4273 75.1161) (end 222.9511 75.1161) (width 0.2) (layer "F.Cu") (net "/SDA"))
 (via (at 221.4273 75.1161) (size 0.6) (drill 0.3) (layers "F.Cu" "B.Cu") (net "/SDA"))
 (segment (start 222.0865 75.7753) (end 222.0865 92.7211) (width 0.2) (layer "B.Cu") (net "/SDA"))
 (segment (start 218.9899 103.1099) (end 220.5 104.62) (width 0.2) (layer "B.Cu") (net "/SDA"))
 (segment (start 221.4273 75.1161) (end 222.0865 75.7753) (width 0.2) (layer "B.Cu") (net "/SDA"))
 (segment (start 218.9899 95.8177) (end 218.9899 103.1099) (width 0.2) (layer "B.Cu") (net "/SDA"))
 (segment (start 222.0865 92.7211) (end 218.9899 95.8177) (width 0.2) (layer "B.Cu") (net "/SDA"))
 (segment (start 223.2922 78.0828) (end 223.335 78.04) (width 0.2) (layer "F.Cu") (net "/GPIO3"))
 (segment (start 221.4173 78.0828) (end 223.2922 78.0828) (width 0.2) (layer "F.Cu") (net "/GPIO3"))
 (via (at 221.4173 78.0828) (size 0.6) (drill 0.3) (layers "F.Cu" "B.Cu") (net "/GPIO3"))
 (segment (start 220.502 78.9981) (end 220.502 84.6418) (width 0.2) (layer "B.Cu") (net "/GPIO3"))
 (segment (start 221.4173 78.0828) (end 220.502 78.9981) (width 0.2) (layer "B.Cu") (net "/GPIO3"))
 (segment (start 204.6438 100.5) (end 193 100.5) (width 0.2) (layer "B.Cu") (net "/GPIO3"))
 (segment (start 220.502 84.6418) (end 204.6438 100.5) (width 0.2) (layer "B.Cu") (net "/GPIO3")))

